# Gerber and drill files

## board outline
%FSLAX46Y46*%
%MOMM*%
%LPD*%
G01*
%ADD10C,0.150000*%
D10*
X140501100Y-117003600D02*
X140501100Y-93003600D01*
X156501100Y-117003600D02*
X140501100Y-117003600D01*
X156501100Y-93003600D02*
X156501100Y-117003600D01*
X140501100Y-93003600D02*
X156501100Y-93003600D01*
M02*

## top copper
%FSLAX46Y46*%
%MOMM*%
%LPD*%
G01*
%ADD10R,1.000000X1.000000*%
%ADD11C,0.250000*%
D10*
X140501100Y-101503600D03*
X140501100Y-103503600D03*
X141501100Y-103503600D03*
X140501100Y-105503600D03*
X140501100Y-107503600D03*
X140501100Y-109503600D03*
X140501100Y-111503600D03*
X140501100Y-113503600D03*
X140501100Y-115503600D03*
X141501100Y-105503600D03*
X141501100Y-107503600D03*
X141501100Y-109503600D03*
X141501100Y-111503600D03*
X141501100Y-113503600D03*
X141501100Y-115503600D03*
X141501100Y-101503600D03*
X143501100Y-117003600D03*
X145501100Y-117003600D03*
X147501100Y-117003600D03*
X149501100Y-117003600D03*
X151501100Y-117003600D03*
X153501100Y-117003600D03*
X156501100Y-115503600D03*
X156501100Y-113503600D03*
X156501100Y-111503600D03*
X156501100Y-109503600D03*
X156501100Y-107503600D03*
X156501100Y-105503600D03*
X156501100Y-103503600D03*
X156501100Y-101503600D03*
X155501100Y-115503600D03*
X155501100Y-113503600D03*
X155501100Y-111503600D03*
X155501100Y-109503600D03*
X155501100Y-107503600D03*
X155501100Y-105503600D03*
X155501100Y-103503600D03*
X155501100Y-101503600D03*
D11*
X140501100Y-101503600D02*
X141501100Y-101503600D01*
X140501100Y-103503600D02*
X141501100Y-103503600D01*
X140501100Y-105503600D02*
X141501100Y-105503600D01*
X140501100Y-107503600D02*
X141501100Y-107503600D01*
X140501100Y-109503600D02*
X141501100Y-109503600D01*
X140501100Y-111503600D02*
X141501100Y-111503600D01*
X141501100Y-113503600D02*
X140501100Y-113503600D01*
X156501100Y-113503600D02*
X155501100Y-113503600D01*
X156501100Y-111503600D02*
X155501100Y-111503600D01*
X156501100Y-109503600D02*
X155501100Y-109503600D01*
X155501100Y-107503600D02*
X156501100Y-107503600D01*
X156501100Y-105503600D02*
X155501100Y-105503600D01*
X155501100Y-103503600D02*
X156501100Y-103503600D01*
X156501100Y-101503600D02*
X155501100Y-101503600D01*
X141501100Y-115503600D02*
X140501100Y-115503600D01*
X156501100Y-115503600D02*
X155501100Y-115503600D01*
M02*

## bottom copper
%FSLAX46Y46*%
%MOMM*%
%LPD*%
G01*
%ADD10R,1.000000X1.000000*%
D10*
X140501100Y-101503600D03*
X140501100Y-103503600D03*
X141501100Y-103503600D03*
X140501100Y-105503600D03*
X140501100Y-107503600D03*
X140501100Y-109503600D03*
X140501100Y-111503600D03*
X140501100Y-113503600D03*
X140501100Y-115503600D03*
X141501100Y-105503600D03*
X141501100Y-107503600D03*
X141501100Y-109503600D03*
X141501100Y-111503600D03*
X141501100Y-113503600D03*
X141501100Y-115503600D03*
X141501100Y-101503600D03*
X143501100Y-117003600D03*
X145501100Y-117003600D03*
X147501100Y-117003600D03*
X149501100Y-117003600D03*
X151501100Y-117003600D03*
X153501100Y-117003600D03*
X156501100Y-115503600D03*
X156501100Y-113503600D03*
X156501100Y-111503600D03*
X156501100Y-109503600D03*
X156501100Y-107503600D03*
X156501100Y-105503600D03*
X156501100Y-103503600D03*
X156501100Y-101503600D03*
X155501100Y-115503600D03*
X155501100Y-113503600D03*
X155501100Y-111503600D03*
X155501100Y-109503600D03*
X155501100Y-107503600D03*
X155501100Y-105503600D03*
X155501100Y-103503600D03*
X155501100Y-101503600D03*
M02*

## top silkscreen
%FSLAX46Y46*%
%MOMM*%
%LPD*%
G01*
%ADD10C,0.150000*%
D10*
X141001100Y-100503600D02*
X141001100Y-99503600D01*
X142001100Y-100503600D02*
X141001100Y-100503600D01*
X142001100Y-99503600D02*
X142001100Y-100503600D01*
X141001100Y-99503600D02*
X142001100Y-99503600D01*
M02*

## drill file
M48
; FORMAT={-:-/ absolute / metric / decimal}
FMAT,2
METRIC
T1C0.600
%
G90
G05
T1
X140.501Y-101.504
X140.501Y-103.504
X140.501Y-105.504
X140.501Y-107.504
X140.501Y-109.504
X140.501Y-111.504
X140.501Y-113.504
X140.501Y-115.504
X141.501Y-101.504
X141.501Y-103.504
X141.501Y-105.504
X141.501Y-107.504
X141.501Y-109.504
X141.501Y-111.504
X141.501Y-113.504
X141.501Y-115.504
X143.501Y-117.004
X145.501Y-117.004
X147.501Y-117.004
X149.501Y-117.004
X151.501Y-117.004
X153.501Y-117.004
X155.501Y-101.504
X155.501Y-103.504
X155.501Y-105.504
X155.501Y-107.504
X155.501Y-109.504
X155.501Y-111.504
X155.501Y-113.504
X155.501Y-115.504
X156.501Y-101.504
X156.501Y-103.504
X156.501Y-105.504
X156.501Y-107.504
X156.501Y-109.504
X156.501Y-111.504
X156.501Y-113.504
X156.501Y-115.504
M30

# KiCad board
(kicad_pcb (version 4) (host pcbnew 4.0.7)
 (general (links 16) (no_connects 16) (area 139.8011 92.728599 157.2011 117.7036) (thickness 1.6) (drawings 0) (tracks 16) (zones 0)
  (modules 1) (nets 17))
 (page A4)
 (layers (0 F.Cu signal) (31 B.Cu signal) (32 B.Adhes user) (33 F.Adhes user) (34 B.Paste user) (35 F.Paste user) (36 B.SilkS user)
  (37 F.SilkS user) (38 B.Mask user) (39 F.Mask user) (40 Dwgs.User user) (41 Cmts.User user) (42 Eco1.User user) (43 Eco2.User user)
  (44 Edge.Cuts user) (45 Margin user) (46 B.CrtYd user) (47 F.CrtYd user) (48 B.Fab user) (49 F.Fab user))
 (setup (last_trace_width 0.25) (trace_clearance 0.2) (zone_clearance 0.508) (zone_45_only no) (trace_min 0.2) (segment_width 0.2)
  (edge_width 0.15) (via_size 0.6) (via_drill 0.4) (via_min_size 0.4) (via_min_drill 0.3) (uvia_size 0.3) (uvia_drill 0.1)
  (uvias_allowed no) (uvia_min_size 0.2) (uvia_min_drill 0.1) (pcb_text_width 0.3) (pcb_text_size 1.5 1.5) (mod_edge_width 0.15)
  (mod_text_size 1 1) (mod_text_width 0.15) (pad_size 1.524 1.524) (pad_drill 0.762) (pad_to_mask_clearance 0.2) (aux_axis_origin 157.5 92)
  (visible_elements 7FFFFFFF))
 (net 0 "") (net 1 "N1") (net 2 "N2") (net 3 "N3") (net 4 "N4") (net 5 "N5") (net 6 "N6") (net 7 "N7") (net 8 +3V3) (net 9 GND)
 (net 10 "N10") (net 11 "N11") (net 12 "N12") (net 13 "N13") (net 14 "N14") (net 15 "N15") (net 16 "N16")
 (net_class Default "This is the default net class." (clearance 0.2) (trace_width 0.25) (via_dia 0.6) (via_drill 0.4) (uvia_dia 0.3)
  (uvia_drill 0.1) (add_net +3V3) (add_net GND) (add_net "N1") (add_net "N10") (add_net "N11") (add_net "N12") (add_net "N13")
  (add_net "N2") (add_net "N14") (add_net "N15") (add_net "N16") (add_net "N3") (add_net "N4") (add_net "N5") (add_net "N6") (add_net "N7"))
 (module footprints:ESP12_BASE (layer F.Cu) (at 148.5011 105.0036)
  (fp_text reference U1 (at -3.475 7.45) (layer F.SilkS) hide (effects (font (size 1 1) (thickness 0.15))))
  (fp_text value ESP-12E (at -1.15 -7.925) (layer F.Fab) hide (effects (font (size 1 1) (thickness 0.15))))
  (fp_line (start -7.5 -4.5) (end -7.5 -5.5) (layer F.SilkS) (width 0.15))
  (fp_line (start -6.5 -4.5) (end -7.5 -4.5) (layer F.SilkS) (width 0.15))
  (fp_line (start -6.5 -5.5) (end -6.5 -4.5) (layer F.SilkS) (width 0.15))
  (fp_line (start -7.5 -5.5) (end -6.5 -5.5) (layer F.SilkS) (width 0.15))
  (fp_line (start -8 12) (end -8 -12) (layer Edge.Cuts) (width 0.15))
  (fp_line (start 8 12) (end -8 12) (layer Edge.Cuts) (width 0.15))
  (fp_line (start 8 -12) (end 8 12) (layer Edge.Cuts) (width 0.15))
  (fp_line (start -8 -12) (end 8 -12) (layer Edge.Cuts) (width 0.15))
  (pad 1 thru_hole rect (at -8 -3.5) (size 1 1) (drill 0.6) (layers *.Cu *.Mask) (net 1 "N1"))
  (pad 2 thru_hole rect (at -8 -1.5) (size 1 1) (drill 0.6) (layers *.Cu *.Mask) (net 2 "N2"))
  (pad 2 thru_hole rect (at -7 -1.5) (size 1 1) (drill 0.6) (layers *.Cu *.Mask) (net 2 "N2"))
  (pad 3 thru_hole rect (at -8 0.5) (size 1 1) (drill 0.6) (layers *.Cu *.Mask) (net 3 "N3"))
  (pad 4 thru_hole rect (at -8 2.5) (size 1 1) (drill 0.6) (layers *.Cu *.Mask) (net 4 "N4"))
  (pad 5 thru_hole rect (at -8 4.5) (size 1 1) (drill 0.6) (layers *.Cu *.Mask) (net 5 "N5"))
  (pad 6 thru_hole rect (at -8 6.5) (size 1 1) (drill 0.6) (layers *.Cu *.Mask) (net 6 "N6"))
  (pad 7 thru_hole rect (at -8 8.5) (size 1 1) (drill 0.6) (layers *.Cu *.Mask) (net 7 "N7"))
  (pad 8 thru_hole rect (at -8 10.5) (size 1 1) (drill 0.6) (layers *.Cu *.Mask) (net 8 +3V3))
  (pad 3 thru_hole rect (at -7 0.5) (size 1 1) (drill 0.6) (layers *.Cu *.Mask) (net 3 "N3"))
  (pad 4 thru_hole rect (at -7 2.5) (size 1 1) (drill 0.6) (layers *.Cu *.Mask) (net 4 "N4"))
  (pad 5 thru_hole rect (at -7 4.5) (size 1 1) (drill 0.6) (layers *.Cu *.Mask) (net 5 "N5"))
  (pad 6 thru_hole rect (at -7 6.5) (size 1 1) (drill 0.6) (layers *.Cu *.Mask) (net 6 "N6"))
  (pad 7 thru_hole rect (at -7 8.5) (size 1 1) (drill 0.6) (layers *.Cu *.Mask) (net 7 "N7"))
  (pad 8 thru_hole rect (at -7 10.5) (size 1 1) (drill 0.6) (layers *.Cu *.Mask) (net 8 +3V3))
  (pad 1 thru_hole rect (at -7 -3.5) (size 1 1) (drill 0.6) (layers *.Cu *.Mask) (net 1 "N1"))
  (pad 9 thru_hole rect (at -5 12) (size 1 1) (drill 0.6) (layers *.Cu *.Mask))
  (pad 10 thru_hole rect (at -3 12) (size 1 1) (drill 0.6) (layers *.Cu *.Mask))
  (pad 11 thru_hole rect (at -1 12) (size 1 1) (drill 0.6) (layers *.Cu *.Mask))
  (pad 12 thru_hole rect (at 1 12) (size 1 1) (drill 0.6) (layers *.Cu *.Mask))
  (pad 13 thru_hole rect (at 3 12) (size 1 1) (drill 0.6) (layers *.Cu *.Mask))
  (pad 14 thru_hole rect (at 5 12) (size 1 1) (drill 0.6) (layers *.Cu *.Mask))
  (pad 15 thru_hole rect (at 8 10.5) (size 1 1) (drill 0.6) (layers *.Cu *.Mask) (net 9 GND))
  (pad 16 thru_hole rect (at 8 8.5) (size 1 1) (drill 0.6) (layers *.Cu *.Mask) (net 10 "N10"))
  (pad 17 thru_hole rect (at 8 6.5) (size 1 1) (drill 0.6) (layers *.Cu *.Mask) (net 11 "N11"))
  (pad 18 thru_hole rect (at 8 4.5) (size 1 1) (drill 0.6) (layers *.Cu *.Mask) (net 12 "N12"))
  (pad 19 thru_hole rect (at 8 2.5) (size 1 1) (drill 0.6) (layers *.Cu *.Mask) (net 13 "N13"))
  (pad 20 thru_hole rect (at 8 0.5) (size 1 1) (drill 0.6) (layers *.Cu *.Mask) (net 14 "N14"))
  (pad 21 thru_hole rect (at 8 -1.5) (size 1 1) (drill 0.6) (layers *.Cu *.Mask) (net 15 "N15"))
  (pad 22 thru_hole rect (at 8 -3.5) (size 1 1) (drill 0.6) (layers *.Cu *.Mask) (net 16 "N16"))
  (pad 15 thru_hole rect (at 7 10.5) (size 1 1) (drill 0.6) (layers *.Cu *.Mask) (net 9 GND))
  (pad 16 thru_hole rect (at 7 8.5) (size 1 1) (drill 0.6) (layers *.Cu *.Mask) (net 10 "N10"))
  (pad 17 thru_hole rect (at 7 6.5) (size 1 1) (drill 0.6) (layers *.Cu *.Mask) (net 11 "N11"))
  (pad 18 thru_hole rect (at 7 4.5) (size 1 1) (drill 0.6) (layers *.Cu *.Mask) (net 12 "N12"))
  (pad 19 thru_hole rect (at 7 2.5) (size 1 1) (drill 0.6) (layers *.Cu *.Mask) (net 13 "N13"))
  (pad 20 thru_hole rect (at 7 0.5) (size 1 1) (drill 0.6) (layers *.Cu *.Mask) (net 14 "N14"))
  (pad 21 thru_hole rect (at 7 -1.5) (size 1 1) (drill 0.6) (layers *.Cu *.Mask) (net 15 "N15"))
  (pad 22 thru_hole rect (at 7 -3.5) (size 1 1) (drill 0.6) (layers *.Cu *.Mask) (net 16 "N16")))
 (segment (start 140.5011 101.5036) (end 141.5011 101.5036) (width 0.25) (layer F.Cu) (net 1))
 (segment (start 140.5011 103.5036) (end 141.5011 103.5036) (width 0.25) (layer F.Cu) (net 2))
 (segment (start 140.5011 105.5036) (end 141.5011 105.5036) (width 0.25) (layer F.Cu) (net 3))
 (segment (start 140.5011 107.5036) (end 141.5011 107.5036) (width 0.25) (layer F.Cu) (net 4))
 (segment (start 140.5011 109.5036) (end 141.5011 109.5036) (width 0.25) (layer F.Cu) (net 5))
 (segment (start 140.5011 111.5036) (end 141.5011 111.5036) (width 0.25) (layer F.Cu) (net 6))
 (segment (start 141.5011 113.5036) (end 140.5011 113.5036) (width 0.25) (layer F.Cu) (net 7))
 (segment (start 156.5011 113.5036) (end 155.5011 113.5036) (width 0.25) (layer F.Cu) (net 10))
 (segment (start 156.5011 111.5036) (end 155.5011 111.5036) (width 0.25) (layer F.Cu) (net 11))
 (segment (start 156.5011 109.5036) (end 155.5011 109.5036) (width 0.25) (layer F.Cu) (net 12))
 (segment (start 155.5011 107.5036) (end 156.5011 107.5036) (width 0.25) (layer F.Cu) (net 13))
 (segment (start 156.5011 105.5036) (end 155.5011 105.5036) (width 0.25) (layer F.Cu) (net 14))
 (segment (start 155.5011 103.5036) (end 156.5011 103.5036) (width 0.25) (layer F.Cu) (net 15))
 (segment (start 156.5011 101.5036) (end 155.5011 101.5036) (width 0.25) (layer F.Cu) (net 16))
 (segment (start 141.5011 115.5036) (end 140.5011 115.5036) (width 0.25) (layer F.Cu) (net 8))
 (segment (start 156.5011 115.5036) (end 155.5011 115.5036) (width 0.25) (layer F.Cu) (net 9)))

